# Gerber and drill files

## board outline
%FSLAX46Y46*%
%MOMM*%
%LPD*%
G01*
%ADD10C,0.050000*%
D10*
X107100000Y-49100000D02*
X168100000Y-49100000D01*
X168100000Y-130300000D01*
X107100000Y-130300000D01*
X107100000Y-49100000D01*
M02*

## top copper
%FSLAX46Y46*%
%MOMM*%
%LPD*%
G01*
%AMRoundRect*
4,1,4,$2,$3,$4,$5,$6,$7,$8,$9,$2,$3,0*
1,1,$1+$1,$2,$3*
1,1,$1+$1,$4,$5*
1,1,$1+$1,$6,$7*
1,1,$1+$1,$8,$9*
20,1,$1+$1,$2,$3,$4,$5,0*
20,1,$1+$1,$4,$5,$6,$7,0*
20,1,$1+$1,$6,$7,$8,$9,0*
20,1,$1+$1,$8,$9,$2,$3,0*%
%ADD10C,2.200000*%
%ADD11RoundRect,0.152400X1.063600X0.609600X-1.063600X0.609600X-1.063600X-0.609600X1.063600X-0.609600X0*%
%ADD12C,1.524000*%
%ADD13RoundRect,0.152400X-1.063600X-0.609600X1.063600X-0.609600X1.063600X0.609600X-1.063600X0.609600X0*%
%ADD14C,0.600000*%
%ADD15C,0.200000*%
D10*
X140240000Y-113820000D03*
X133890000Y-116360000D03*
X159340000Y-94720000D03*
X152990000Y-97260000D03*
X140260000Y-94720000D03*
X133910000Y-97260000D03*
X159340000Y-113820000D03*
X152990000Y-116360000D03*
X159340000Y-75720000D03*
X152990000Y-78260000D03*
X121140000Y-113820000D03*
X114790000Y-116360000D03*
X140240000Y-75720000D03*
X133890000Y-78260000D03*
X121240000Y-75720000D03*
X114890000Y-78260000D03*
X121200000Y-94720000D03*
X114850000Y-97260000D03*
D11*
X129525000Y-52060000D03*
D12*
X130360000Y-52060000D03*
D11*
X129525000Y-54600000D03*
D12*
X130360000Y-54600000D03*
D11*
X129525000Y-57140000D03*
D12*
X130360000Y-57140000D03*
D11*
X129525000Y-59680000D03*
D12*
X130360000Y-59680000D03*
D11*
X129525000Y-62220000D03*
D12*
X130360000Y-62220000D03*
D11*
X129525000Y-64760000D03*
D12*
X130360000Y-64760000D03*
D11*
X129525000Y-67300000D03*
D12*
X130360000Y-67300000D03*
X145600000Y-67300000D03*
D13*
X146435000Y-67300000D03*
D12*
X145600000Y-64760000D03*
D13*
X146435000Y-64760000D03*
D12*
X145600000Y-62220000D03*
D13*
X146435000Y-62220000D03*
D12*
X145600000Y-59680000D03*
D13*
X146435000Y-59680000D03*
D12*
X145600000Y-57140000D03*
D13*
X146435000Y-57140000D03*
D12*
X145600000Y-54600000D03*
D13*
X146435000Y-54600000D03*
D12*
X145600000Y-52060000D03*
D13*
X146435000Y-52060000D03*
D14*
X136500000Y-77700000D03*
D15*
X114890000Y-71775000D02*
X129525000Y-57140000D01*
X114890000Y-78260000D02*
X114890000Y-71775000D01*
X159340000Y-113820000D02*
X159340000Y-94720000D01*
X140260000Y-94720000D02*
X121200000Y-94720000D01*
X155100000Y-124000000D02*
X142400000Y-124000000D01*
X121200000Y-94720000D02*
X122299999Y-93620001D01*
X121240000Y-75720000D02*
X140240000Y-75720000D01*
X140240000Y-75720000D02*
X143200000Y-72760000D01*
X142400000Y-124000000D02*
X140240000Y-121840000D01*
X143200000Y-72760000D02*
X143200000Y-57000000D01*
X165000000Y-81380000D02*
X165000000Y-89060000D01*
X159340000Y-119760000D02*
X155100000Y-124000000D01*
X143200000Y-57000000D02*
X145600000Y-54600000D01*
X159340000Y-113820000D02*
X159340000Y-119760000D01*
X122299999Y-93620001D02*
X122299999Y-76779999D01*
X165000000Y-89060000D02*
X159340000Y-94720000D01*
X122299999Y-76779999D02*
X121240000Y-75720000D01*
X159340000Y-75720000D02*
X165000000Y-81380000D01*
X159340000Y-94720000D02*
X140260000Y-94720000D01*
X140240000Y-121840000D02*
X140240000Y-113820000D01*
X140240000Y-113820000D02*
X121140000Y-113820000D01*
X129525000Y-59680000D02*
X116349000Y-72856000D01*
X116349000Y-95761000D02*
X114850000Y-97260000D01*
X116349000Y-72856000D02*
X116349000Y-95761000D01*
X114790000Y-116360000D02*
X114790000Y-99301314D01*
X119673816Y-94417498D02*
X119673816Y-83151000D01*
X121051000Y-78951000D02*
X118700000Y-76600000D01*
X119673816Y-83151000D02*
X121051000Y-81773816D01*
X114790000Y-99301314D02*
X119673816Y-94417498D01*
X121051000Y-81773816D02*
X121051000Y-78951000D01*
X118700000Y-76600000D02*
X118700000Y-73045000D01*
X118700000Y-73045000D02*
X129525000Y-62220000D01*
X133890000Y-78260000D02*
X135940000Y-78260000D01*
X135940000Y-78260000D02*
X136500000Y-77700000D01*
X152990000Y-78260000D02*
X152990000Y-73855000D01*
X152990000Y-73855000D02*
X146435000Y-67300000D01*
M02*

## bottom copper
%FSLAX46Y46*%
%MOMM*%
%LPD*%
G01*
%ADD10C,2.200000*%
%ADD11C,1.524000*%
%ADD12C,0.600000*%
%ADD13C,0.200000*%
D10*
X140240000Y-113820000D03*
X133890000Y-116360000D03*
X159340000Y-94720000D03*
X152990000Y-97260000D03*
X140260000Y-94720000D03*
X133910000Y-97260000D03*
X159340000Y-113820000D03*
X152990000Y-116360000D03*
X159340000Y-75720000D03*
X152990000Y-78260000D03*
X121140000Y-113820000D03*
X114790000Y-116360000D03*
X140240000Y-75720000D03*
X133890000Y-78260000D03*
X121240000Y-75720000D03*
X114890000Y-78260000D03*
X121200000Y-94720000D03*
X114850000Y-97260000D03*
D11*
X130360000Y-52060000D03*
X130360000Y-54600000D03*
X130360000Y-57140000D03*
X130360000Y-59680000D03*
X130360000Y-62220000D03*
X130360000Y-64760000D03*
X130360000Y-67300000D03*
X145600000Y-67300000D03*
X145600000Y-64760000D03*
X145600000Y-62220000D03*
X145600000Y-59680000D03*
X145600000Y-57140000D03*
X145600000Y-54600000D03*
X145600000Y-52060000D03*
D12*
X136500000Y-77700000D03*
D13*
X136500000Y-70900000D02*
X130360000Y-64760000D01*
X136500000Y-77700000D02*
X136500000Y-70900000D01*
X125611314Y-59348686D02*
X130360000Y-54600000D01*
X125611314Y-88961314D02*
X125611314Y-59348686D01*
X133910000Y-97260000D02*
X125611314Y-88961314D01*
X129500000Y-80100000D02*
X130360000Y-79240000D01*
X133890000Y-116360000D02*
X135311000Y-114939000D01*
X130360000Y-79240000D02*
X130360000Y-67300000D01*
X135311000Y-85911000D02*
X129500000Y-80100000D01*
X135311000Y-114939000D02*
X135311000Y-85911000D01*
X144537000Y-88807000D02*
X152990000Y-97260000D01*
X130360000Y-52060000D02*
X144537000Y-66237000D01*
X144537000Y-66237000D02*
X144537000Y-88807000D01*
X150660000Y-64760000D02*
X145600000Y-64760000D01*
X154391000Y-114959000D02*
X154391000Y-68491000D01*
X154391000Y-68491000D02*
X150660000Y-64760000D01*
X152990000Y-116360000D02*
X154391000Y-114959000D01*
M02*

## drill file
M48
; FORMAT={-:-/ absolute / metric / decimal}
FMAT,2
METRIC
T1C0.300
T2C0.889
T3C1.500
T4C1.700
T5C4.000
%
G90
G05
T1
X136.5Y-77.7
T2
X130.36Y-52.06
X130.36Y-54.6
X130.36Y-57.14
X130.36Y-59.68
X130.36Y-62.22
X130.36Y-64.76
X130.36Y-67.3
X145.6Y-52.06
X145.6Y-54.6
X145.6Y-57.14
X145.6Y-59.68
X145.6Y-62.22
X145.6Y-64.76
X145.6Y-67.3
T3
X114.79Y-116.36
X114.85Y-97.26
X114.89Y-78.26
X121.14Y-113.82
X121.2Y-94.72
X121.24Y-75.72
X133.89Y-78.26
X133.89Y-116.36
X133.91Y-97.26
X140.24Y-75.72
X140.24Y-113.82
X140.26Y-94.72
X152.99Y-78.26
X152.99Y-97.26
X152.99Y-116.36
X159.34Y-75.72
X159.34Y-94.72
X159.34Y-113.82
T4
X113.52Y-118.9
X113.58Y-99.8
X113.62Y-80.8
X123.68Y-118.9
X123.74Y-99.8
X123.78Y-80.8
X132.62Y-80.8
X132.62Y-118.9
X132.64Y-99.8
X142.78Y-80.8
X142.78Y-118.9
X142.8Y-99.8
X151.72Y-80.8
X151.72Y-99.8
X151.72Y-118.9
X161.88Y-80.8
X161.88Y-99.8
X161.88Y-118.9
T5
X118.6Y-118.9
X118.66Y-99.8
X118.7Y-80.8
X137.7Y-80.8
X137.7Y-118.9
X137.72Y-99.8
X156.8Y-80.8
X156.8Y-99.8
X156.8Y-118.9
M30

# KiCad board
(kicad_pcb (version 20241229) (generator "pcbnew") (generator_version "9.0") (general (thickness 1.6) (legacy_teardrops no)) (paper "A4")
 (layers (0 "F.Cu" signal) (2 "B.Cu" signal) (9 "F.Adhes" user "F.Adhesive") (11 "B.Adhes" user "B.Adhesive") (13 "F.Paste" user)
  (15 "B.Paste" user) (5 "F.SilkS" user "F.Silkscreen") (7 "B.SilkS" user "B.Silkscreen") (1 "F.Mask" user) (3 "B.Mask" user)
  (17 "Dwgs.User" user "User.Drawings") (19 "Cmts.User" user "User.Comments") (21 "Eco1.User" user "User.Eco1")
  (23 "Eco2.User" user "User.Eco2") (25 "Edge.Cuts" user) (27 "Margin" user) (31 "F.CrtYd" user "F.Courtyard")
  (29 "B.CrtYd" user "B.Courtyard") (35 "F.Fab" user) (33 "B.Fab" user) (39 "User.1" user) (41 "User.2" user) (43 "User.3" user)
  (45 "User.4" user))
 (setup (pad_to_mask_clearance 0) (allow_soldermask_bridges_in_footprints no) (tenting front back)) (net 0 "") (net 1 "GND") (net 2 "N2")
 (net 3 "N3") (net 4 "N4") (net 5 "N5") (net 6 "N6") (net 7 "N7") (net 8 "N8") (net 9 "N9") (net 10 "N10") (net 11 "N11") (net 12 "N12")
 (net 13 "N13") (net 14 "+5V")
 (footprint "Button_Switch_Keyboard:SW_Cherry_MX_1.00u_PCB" (layer "F.Cu") (at 140.24 113.82)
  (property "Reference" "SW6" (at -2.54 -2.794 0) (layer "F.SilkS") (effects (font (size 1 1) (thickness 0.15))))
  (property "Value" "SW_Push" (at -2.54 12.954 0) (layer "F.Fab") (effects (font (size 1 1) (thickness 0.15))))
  (pad "" np_thru_hole circle (at -7.62 5.08) (size 1.7 1.7) (drill 1.7) (layers "*.Cu" "*.Mask"))
  (pad "" np_thru_hole circle (at -2.54 5.08) (size 4 4) (drill 4) (layers "*.Cu" "*.Mask"))
  (pad "" np_thru_hole circle (at 2.54 5.08) (size 1.7 1.7) (drill 1.7) (layers "*.Cu" "*.Mask"))
  (pad "1" thru_hole circle (at 0 0) (size 2.2 2.2) (drill 1.5) (layers "*.Cu" "*.Mask") (remove_unused_layers no) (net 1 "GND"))
  (pad "2" thru_hole circle (at -6.35 2.54) (size 2.2 2.2) (drill 1.5) (layers "*.Cu" "*.Mask") (remove_unused_layers no) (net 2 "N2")))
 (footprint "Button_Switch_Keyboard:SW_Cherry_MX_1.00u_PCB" (layer "F.Cu") (at 159.34 94.72)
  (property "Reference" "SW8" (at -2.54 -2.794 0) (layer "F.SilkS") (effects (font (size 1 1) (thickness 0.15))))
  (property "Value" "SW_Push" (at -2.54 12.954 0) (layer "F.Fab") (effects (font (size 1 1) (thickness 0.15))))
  (pad "" np_thru_hole circle (at -7.62 5.08) (size 1.7 1.7) (drill 1.7) (layers "*.Cu" "*.Mask"))
  (pad "" np_thru_hole circle (at -2.54 5.08) (size 4 4) (drill 4) (layers "*.Cu" "*.Mask"))
  (pad "" np_thru_hole circle (at 2.54 5.08) (size 1.7 1.7) (drill 1.7) (layers "*.Cu" "*.Mask"))
  (pad "1" thru_hole circle (at 0 0) (size 2.2 2.2) (drill 1.5) (layers "*.Cu" "*.Mask") (remove_unused_layers no) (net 1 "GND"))
  (pad "2" thru_hole circle (at -6.35 2.54) (size 2.2 2.2) (drill 1.5) (layers "*.Cu" "*.Mask") (remove_unused_layers no) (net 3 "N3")))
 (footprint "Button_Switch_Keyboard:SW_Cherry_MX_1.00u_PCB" (layer "F.Cu") (at 140.26 94.72)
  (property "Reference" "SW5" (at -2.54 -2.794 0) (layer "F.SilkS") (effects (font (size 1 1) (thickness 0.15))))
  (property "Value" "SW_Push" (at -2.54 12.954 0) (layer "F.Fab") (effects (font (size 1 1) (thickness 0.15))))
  (pad "" np_thru_hole circle (at -7.62 5.08) (size 1.7 1.7) (drill 1.7) (layers "*.Cu" "*.Mask"))
  (pad "" np_thru_hole circle (at -2.54 5.08) (size 4 4) (drill 4) (layers "*.Cu" "*.Mask"))
  (pad "" np_thru_hole circle (at 2.54 5.08) (size 1.7 1.7) (drill 1.7) (layers "*.Cu" "*.Mask"))
  (pad "1" thru_hole circle (at 0 0) (size 2.2 2.2) (drill 1.5) (layers "*.Cu" "*.Mask") (remove_unused_layers no) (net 1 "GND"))
  (pad "2" thru_hole circle (at -6.35 2.54) (size 2.2 2.2) (drill 1.5) (layers "*.Cu" "*.Mask") (remove_unused_layers no) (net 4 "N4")))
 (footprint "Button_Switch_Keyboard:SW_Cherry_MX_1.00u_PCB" (layer "F.Cu") (at 159.34 113.82)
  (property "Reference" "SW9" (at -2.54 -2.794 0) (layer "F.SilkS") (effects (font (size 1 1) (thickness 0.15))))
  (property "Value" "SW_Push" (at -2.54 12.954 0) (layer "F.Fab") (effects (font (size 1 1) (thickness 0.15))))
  (pad "" np_thru_hole circle (at -7.62 5.08) (size 1.7 1.7) (drill 1.7) (layers "*.Cu" "*.Mask"))
  (pad "" np_thru_hole circle (at -2.54 5.08) (size 4 4) (drill 4) (layers "*.Cu" "*.Mask"))
  (pad "" np_thru_hole circle (at 2.54 5.08) (size 1.7 1.7) (drill 1.7) (layers "*.Cu" "*.Mask"))
  (pad "1" thru_hole circle (at 0 0) (size 2.2 2.2) (drill 1.5) (layers "*.Cu" "*.Mask") (remove_unused_layers no) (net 1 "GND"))
  (pad "2" thru_hole circle (at -6.35 2.54) (size 2.2 2.2) (drill 1.5) (layers "*.Cu" "*.Mask") (remove_unused_layers no) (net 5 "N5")))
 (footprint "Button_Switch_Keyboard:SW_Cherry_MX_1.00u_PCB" (layer "F.Cu") (at 159.34 75.72)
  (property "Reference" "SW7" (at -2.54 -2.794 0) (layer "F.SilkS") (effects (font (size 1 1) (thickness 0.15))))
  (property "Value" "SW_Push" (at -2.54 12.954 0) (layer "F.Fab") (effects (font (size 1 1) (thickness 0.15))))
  (pad "" np_thru_hole circle (at -7.62 5.08) (size 1.7 1.7) (drill 1.7) (layers "*.Cu" "*.Mask"))
  (pad "" np_thru_hole circle (at -2.54 5.08) (size 4 4) (drill 4) (layers "*.Cu" "*.Mask"))
  (pad "" np_thru_hole circle (at 2.54 5.08) (size 1.7 1.7) (drill 1.7) (layers "*.Cu" "*.Mask"))
  (pad "1" thru_hole circle (at 0 0) (size 2.2 2.2) (drill 1.5) (layers "*.Cu" "*.Mask") (remove_unused_layers no) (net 1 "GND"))
  (pad "2" thru_hole circle (at -6.35 2.54) (size 2.2 2.2) (drill 1.5) (layers "*.Cu" "*.Mask") (remove_unused_layers no) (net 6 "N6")))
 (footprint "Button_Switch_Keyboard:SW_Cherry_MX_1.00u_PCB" (layer "F.Cu") (at 121.14 113.82)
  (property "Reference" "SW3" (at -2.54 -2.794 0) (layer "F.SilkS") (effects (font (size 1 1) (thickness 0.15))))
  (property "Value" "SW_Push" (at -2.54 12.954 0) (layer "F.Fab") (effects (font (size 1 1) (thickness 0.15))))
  (pad "" np_thru_hole circle (at -7.62 5.08) (size 1.7 1.7) (drill 1.7) (layers "*.Cu" "*.Mask"))
  (pad "" np_thru_hole circle (at -2.54 5.08) (size 4 4) (drill 4) (layers "*.Cu" "*.Mask"))
  (pad "" np_thru_hole circle (at 2.54 5.08) (size 1.7 1.7) (drill 1.7) (layers "*.Cu" "*.Mask"))
  (pad "1" thru_hole circle (at 0 0) (size 2.2 2.2) (drill 1.5) (layers "*.Cu" "*.Mask") (remove_unused_layers no) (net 1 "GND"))
  (pad "2" thru_hole circle (at -6.35 2.54) (size 2.2 2.2) (drill 1.5) (layers "*.Cu" "*.Mask") (remove_unused_layers no) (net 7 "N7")))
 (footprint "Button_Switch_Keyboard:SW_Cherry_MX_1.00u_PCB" (layer "F.Cu") (at 140.24 75.72)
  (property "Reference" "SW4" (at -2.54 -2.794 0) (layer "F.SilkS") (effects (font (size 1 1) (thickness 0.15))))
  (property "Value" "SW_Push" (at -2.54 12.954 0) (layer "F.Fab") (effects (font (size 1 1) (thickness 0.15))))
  (pad "" np_thru_hole circle (at -7.62 5.08) (size 1.7 1.7) (drill 1.7) (layers "*.Cu" "*.Mask"))
  (pad "" np_thru_hole circle (at -2.54 5.08) (size 4 4) (drill 4) (layers "*.Cu" "*.Mask"))
  (pad "" np_thru_hole circle (at 2.54 5.08) (size 1.7 1.7) (drill 1.7) (layers "*.Cu" "*.Mask"))
  (pad "1" thru_hole circle (at 0 0) (size 2.2 2.2) (drill 1.5) (layers "*.Cu" "*.Mask") (remove_unused_layers no) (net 1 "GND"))
  (pad "2" thru_hole circle (at -6.35 2.54) (size 2.2 2.2) (drill 1.5) (layers "*.Cu" "*.Mask") (remove_unused_layers no) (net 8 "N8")))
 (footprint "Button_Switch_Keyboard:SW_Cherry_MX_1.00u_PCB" (layer "F.Cu") (at 121.24 75.72)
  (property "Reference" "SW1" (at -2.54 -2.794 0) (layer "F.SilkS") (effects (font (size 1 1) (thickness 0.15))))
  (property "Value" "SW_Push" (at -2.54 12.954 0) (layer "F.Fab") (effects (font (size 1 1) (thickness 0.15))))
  (pad "" np_thru_hole circle (at -7.62 5.08) (size 1.7 1.7) (drill 1.7) (layers "*.Cu" "*.Mask"))
  (pad "" np_thru_hole circle (at -2.54 5.08) (size 4 4) (drill 4) (layers "*.Cu" "*.Mask"))
  (pad "" np_thru_hole circle (at 2.54 5.08) (size 1.7 1.7) (drill 1.7) (layers "*.Cu" "*.Mask"))
  (pad "1" thru_hole circle (at 0 0) (size 2.2 2.2) (drill 1.5) (layers "*.Cu" "*.Mask") (remove_unused_layers no) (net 1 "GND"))
  (pad "2" thru_hole circle (at -6.35 2.54) (size 2.2 2.2) (drill 1.5) (layers "*.Cu" "*.Mask") (remove_unused_layers no) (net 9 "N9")))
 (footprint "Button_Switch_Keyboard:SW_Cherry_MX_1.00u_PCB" (layer "F.Cu") (at 121.2 94.72)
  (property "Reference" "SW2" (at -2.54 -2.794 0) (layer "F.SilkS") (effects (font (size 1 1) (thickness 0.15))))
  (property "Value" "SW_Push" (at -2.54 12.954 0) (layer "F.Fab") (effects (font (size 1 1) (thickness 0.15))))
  (pad "" np_thru_hole circle (at -7.62 5.08) (size 1.7 1.7) (drill 1.7) (layers "*.Cu" "*.Mask"))
  (pad "" np_thru_hole circle (at -2.54 5.08) (size 4 4) (drill 4) (layers "*.Cu" "*.Mask"))
  (pad "" np_thru_hole circle (at 2.54 5.08) (size 1.7 1.7) (drill 1.7) (layers "*.Cu" "*.Mask"))
  (pad "1" thru_hole circle (at 0 0) (size 2.2 2.2) (drill 1.5) (layers "*.Cu" "*.Mask") (remove_unused_layers no) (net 1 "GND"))
  (pad "2" thru_hole circle (at -6.35 2.54) (size 2.2 2.2) (drill 1.5) (layers "*.Cu" "*.Mask") (remove_unused_layers no) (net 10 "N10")))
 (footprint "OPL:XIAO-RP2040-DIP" (layer "F.Cu") (at 137.98 59.68)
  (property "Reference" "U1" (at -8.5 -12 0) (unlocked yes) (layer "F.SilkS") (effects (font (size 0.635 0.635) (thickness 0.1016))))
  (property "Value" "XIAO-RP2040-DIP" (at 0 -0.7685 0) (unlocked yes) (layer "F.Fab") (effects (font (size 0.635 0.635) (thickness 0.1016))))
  (pad "1" smd roundrect (at -8.455 -7.62 180) (size 2.432 1.524) (layers "F.Cu" "F.Mask") (roundrect_rratio 0.1) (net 3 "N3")
   (thermal_bridge_angle 45))
  (pad "1" thru_hole circle (at -7.62 -7.62 180) (size 1.524 1.524) (drill 0.889) (layers "*.Cu" "*.Mask") (remove_unused_layers no)
   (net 3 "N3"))
  (pad "2" smd roundrect (at -8.455 -5.08 180) (size 2.432 1.524) (layers "F.Cu" "F.Mask") (roundrect_rratio 0.1) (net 4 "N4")
   (thermal_bridge_angle 45))
  (pad "2" thru_hole circle (at -7.62 -5.08 180) (size 1.524 1.524) (drill 0.889) (layers "*.Cu" "*.Mask") (remove_unused_layers no)
   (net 4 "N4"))
  (pad "3" smd roundrect (at -8.455 -2.54 180) (size 2.432 1.524) (layers "F.Cu" "F.Mask") (roundrect_rratio 0.1) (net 9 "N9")
   (thermal_bridge_angle 45))
  (pad "3" thru_hole circle (at -7.62 -2.54 180) (size 1.524 1.524) (drill 0.889) (layers "*.Cu" "*.Mask") (remove_unused_layers no)
   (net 9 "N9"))
  (pad "4" smd roundrect (at -8.455 0 180) (size 2.432 1.524) (layers "F.Cu" "F.Mask") (roundrect_rratio 0.1) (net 10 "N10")
   (thermal_bridge_angle 45))
  (pad "4" thru_hole circle (at -7.62 0 180) (size 1.524 1.524) (drill 0.889) (layers "*.Cu" "*.Mask") (remove_unused_layers no)
   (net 10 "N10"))
  (pad "5" smd roundrect (at -8.455 2.54 180) (size 2.432 1.524) (layers "F.Cu" "F.Mask") (roundrect_rratio 0.1) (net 7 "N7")
   (thermal_bridge_angle 45))
  (pad "5" thru_hole circle (at -7.62 2.54 180) (size 1.524 1.524) (drill 0.889) (layers "*.Cu" "*.Mask") (remove_unused_layers no)
   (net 7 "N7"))
  (pad "6" smd roundrect (at -8.455 5.08 180) (size 2.432 1.524) (layers "F.Cu" "F.Mask") (roundrect_rratio 0.1) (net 8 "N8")
   (thermal_bridge_angle 45))
  (pad "6" thru_hole circle (at -7.62 5.08 180) (size 1.524 1.524) (drill 0.889) (layers "*.Cu" "*.Mask") (remove_unused_layers no)
   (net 8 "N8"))
  (pad "7" smd roundrect (at -8.455 7.62 180) (size 2.432 1.524) (layers "F.Cu" "F.Mask") (roundrect_rratio 0.1) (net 2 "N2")
   (thermal_bridge_angle 45))
  (pad "7" thru_hole circle (at -7.62 7.62 180) (size 1.524 1.524) (drill 0.889) (layers "*.Cu" "*.Mask") (remove_unused_layers no)
   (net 2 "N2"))
  (pad "8" thru_hole circle (at 7.62 7.62) (size 1.524 1.524) (drill 0.889) (layers "*.Cu" "*.Mask") (remove_unused_layers no) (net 6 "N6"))
  (pad "8" smd roundrect (at 8.455 7.62) (size 2.432 1.524) (layers "F.Cu" "F.Mask") (roundrect_rratio 0.1) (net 6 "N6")
   (thermal_bridge_angle 45))
  (pad "9" thru_hole circle (at 7.62 5.08) (size 1.524 1.524) (drill 0.889) (layers "*.Cu" "*.Mask") (remove_unused_layers no) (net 5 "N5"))
  (pad "9" smd roundrect (at 8.455 5.08) (size 2.432 1.524) (layers "F.Cu" "F.Mask") (roundrect_rratio 0.1) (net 5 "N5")
   (thermal_bridge_angle 45))
  (pad "10" thru_hole circle (at 7.62 2.54) (size 1.524 1.524) (drill 0.889) (layers "*.Cu" "*.Mask") (remove_unused_layers no)
   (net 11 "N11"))
  (pad "10" smd roundrect (at 8.455 2.54) (size 2.432 1.524) (layers "F.Cu" "F.Mask") (roundrect_rratio 0.1) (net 11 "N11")
   (thermal_bridge_angle 45))
  (pad "11" thru_hole circle (at 7.62 0) (size 1.524 1.524) (drill 0.889) (layers "*.Cu" "*.Mask") (remove_unused_layers no) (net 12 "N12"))
  (pad "11" smd roundrect (at 8.455 0) (size 2.432 1.524) (layers "F.Cu" "F.Mask") (roundrect_rratio 0.1) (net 12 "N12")
   (thermal_bridge_angle 45))
  (pad "12" thru_hole circle (at 7.62 -2.54) (size 1.524 1.524) (drill 0.889) (layers "*.Cu" "*.Mask") (remove_unused_layers no)
   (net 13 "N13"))
  (pad "12" smd roundrect (at 8.455 -2.54) (size 2.432 1.524) (layers "F.Cu" "F.Mask") (roundrect_rratio 0.1) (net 13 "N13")
   (thermal_bridge_angle 45))
  (pad "13" thru_hole circle (at 7.62 -5.08) (size 1.524 1.524) (drill 0.889) (layers "*.Cu" "*.Mask") (remove_unused_layers no)
   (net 1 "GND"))
  (pad "13" smd roundrect (at 8.455 -5.08) (size 2.432 1.524) (layers "F.Cu" "F.Mask") (roundrect_rratio 0.1) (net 1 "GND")
   (thermal_bridge_angle 45))
  (pad "14" thru_hole circle (at 7.62 -7.62) (size 1.524 1.524) (drill 0.889) (layers "*.Cu" "*.Mask") (remove_unused_layers no)
   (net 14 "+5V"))
  (pad "14" smd roundrect (at 8.455 -7.62) (size 2.432 1.524) (layers "F.Cu" "F.Mask") (roundrect_rratio 0.1) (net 14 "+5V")
   (thermal_bridge_angle 45)))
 (gr_rect (start 107.1 49.1) (end 168.1 130.3) (stroke (width 0.05) (type default)) (fill no) (layer "Edge.Cuts"))
 (segment (start 114.89 71.775) (end 129.525 57.14) (width 0.2) (layer "F.Cu") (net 9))
 (segment (start 114.89 78.26) (end 114.89 71.775) (width 0.2) (layer "F.Cu") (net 9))
 (segment (start 159.34 113.82) (end 159.34 94.72) (width 0.2) (layer "F.Cu") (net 1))
 (segment (start 140.26 94.72) (end 121.2 94.72) (width 0.2) (layer "F.Cu") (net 1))
 (segment (start 155.1 124) (end 142.4 124) (width 0.2) (layer "F.Cu") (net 1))
 (segment (start 121.2 94.72) (end 122.299999 93.620001) (width 0.2) (layer "F.Cu") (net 1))
 (segment (start 121.24 75.72) (end 140.24 75.72) (width 0.2) (layer "F.Cu") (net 1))
 (segment (start 140.24 75.72) (end 143.2 72.76) (width 0.2) (layer "F.Cu") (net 1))
 (segment (start 142.4 124) (end 140.24 121.84) (width 0.2) (layer "F.Cu") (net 1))
 (segment (start 143.2 72.76) (end 143.2 57) (width 0.2) (layer "F.Cu") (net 1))
 (segment (start 165 81.38) (end 165 89.06) (width 0.2) (layer "F.Cu") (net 1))
 (segment (start 159.34 119.76) (end 155.1 124) (width 0.2) (layer "F.Cu") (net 1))
 (segment (start 143.2 57) (end 145.6 54.6) (width 0.2) (layer "F.Cu") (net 1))
 (segment (start 159.34 113.82) (end 159.34 119.76) (width 0.2) (layer "F.Cu") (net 1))
 (segment (start 122.299999 93.620001) (end 122.299999 76.779999) (width 0.2) (layer "F.Cu") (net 1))
 (segment (start 165 89.06) (end 159.34 94.72) (width 0.2) (layer "F.Cu") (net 1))
 (segment (start 122.299999 76.779999) (end 121.24 75.72) (width 0.2) (layer "F.Cu") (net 1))
 (segment (start 159.34 75.72) (end 165 81.38) (width 0.2) (layer "F.Cu") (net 1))
 (segment (start 159.34 94.72) (end 140.26 94.72) (width 0.2) (layer "F.Cu") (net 1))
 (segment (start 140.24 121.84) (end 140.24 113.82) (width 0.2) (layer "F.Cu") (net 1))
 (segment (start 140.24 113.82) (end 121.14 113.82) (width 0.2) (layer "F.Cu") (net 1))
 (segment (start 129.525 59.68) (end 116.349 72.856) (width 0.2) (layer "F.Cu") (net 10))
 (segment (start 116.349 95.761) (end 114.85 97.26) (width 0.2) (layer "F.Cu") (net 10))
 (segment (start 116.349 72.856) (end 116.349 95.761) (width 0.2) (layer "F.Cu") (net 10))
 (segment (start 114.79 116.36) (end 114.79 99.301314) (width 0.2) (layer "F.Cu") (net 7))
 (segment (start 119.673816 94.417498) (end 119.673816 83.151) (width 0.2) (layer "F.Cu") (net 7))
 (segment (start 121.051 78.951) (end 118.7 76.6) (width 0.2) (layer "F.Cu") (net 7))
 (segment (start 119.673816 83.151) (end 121.051 81.773816) (width 0.2) (layer "F.Cu") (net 7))
 (segment (start 114.79 99.301314) (end 119.673816 94.417498) (width 0.2) (layer "F.Cu") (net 7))
 (segment (start 121.051 81.773816) (end 121.051 78.951) (width 0.2) (layer "F.Cu") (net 7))
 (segment (start 118.7 76.6) (end 118.7 73.045) (width 0.2) (layer "F.Cu") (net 7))
 (segment (start 118.7 73.045) (end 129.525 62.22) (width 0.2) (layer "F.Cu") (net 7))
 (segment (start 133.89 78.26) (end 135.94 78.26) (width 0.2) (layer "F.Cu") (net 8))
 (segment (start 135.94 78.26) (end 136.5 77.7) (width 0.2) (layer "F.Cu") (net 8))
 (via (at 136.5 77.7) (size 0.6) (drill 0.3) (layers "F.Cu" "B.Cu") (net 8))
 (segment (start 136.5 70.9) (end 130.36 64.76) (width 0.2) (layer "B.Cu") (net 8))
 (segment (start 136.5 77.7) (end 136.5 70.9) (width 0.2) (layer "B.Cu") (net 8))
 (segment (start 125.611314 59.348686) (end 130.36 54.6) (width 0.2) (layer "B.Cu") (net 4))
 (segment (start 125.611314 88.961314) (end 125.611314 59.348686) (width 0.2) (layer "B.Cu") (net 4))
 (segment (start 133.91 97.26) (end 125.611314 88.961314) (width 0.2) (layer "B.Cu") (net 4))
 (segment (start 129.5 80.1) (end 130.36 79.24) (width 0.2) (layer "B.Cu") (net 2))
 (segment (start 133.89 116.36) (end 135.311 114.939) (width 0.2) (layer "B.Cu") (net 2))
 (segment (start 130.36 79.24) (end 130.36 67.3) (width 0.2) (layer "B.Cu") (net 2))
 (segment (start 135.311 85.911) (end 129.5 80.1) (width 0.2) (layer "B.Cu") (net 2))
 (segment (start 135.311 114.939) (end 135.311 85.911) (width 0.2) (layer "B.Cu") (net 2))
 (segment (start 152.99 78.26) (end 152.99 73.855) (width 0.2) (layer "F.Cu") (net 6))
 (segment (start 152.99 73.855) (end 146.435 67.3) (width 0.2) (layer "F.Cu") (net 6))
 (segment (start 144.537 88.807) (end 152.99 97.26) (width 0.2) (layer "B.Cu") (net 3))
 (segment (start 130.36 52.06) (end 144.537 66.237) (width 0.2) (layer "B.Cu") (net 3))
 (segment (start 144.537 66.237) (end 144.537 88.807) (width 0.2) (layer "B.Cu") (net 3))
 (segment (start 150.66 64.76) (end 145.6 64.76) (width 0.2) (layer "B.Cu") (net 5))
 (segment (start 154.391 114.959) (end 154.391 68.491) (width 0.2) (layer "B.Cu") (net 5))
 (segment (start 154.391 68.491) (end 150.66 64.76) (width 0.2) (layer "B.Cu") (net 5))
 (segment (start 152.99 116.36) (end 154.391 114.959) (width 0.2) (layer "B.Cu") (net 5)))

